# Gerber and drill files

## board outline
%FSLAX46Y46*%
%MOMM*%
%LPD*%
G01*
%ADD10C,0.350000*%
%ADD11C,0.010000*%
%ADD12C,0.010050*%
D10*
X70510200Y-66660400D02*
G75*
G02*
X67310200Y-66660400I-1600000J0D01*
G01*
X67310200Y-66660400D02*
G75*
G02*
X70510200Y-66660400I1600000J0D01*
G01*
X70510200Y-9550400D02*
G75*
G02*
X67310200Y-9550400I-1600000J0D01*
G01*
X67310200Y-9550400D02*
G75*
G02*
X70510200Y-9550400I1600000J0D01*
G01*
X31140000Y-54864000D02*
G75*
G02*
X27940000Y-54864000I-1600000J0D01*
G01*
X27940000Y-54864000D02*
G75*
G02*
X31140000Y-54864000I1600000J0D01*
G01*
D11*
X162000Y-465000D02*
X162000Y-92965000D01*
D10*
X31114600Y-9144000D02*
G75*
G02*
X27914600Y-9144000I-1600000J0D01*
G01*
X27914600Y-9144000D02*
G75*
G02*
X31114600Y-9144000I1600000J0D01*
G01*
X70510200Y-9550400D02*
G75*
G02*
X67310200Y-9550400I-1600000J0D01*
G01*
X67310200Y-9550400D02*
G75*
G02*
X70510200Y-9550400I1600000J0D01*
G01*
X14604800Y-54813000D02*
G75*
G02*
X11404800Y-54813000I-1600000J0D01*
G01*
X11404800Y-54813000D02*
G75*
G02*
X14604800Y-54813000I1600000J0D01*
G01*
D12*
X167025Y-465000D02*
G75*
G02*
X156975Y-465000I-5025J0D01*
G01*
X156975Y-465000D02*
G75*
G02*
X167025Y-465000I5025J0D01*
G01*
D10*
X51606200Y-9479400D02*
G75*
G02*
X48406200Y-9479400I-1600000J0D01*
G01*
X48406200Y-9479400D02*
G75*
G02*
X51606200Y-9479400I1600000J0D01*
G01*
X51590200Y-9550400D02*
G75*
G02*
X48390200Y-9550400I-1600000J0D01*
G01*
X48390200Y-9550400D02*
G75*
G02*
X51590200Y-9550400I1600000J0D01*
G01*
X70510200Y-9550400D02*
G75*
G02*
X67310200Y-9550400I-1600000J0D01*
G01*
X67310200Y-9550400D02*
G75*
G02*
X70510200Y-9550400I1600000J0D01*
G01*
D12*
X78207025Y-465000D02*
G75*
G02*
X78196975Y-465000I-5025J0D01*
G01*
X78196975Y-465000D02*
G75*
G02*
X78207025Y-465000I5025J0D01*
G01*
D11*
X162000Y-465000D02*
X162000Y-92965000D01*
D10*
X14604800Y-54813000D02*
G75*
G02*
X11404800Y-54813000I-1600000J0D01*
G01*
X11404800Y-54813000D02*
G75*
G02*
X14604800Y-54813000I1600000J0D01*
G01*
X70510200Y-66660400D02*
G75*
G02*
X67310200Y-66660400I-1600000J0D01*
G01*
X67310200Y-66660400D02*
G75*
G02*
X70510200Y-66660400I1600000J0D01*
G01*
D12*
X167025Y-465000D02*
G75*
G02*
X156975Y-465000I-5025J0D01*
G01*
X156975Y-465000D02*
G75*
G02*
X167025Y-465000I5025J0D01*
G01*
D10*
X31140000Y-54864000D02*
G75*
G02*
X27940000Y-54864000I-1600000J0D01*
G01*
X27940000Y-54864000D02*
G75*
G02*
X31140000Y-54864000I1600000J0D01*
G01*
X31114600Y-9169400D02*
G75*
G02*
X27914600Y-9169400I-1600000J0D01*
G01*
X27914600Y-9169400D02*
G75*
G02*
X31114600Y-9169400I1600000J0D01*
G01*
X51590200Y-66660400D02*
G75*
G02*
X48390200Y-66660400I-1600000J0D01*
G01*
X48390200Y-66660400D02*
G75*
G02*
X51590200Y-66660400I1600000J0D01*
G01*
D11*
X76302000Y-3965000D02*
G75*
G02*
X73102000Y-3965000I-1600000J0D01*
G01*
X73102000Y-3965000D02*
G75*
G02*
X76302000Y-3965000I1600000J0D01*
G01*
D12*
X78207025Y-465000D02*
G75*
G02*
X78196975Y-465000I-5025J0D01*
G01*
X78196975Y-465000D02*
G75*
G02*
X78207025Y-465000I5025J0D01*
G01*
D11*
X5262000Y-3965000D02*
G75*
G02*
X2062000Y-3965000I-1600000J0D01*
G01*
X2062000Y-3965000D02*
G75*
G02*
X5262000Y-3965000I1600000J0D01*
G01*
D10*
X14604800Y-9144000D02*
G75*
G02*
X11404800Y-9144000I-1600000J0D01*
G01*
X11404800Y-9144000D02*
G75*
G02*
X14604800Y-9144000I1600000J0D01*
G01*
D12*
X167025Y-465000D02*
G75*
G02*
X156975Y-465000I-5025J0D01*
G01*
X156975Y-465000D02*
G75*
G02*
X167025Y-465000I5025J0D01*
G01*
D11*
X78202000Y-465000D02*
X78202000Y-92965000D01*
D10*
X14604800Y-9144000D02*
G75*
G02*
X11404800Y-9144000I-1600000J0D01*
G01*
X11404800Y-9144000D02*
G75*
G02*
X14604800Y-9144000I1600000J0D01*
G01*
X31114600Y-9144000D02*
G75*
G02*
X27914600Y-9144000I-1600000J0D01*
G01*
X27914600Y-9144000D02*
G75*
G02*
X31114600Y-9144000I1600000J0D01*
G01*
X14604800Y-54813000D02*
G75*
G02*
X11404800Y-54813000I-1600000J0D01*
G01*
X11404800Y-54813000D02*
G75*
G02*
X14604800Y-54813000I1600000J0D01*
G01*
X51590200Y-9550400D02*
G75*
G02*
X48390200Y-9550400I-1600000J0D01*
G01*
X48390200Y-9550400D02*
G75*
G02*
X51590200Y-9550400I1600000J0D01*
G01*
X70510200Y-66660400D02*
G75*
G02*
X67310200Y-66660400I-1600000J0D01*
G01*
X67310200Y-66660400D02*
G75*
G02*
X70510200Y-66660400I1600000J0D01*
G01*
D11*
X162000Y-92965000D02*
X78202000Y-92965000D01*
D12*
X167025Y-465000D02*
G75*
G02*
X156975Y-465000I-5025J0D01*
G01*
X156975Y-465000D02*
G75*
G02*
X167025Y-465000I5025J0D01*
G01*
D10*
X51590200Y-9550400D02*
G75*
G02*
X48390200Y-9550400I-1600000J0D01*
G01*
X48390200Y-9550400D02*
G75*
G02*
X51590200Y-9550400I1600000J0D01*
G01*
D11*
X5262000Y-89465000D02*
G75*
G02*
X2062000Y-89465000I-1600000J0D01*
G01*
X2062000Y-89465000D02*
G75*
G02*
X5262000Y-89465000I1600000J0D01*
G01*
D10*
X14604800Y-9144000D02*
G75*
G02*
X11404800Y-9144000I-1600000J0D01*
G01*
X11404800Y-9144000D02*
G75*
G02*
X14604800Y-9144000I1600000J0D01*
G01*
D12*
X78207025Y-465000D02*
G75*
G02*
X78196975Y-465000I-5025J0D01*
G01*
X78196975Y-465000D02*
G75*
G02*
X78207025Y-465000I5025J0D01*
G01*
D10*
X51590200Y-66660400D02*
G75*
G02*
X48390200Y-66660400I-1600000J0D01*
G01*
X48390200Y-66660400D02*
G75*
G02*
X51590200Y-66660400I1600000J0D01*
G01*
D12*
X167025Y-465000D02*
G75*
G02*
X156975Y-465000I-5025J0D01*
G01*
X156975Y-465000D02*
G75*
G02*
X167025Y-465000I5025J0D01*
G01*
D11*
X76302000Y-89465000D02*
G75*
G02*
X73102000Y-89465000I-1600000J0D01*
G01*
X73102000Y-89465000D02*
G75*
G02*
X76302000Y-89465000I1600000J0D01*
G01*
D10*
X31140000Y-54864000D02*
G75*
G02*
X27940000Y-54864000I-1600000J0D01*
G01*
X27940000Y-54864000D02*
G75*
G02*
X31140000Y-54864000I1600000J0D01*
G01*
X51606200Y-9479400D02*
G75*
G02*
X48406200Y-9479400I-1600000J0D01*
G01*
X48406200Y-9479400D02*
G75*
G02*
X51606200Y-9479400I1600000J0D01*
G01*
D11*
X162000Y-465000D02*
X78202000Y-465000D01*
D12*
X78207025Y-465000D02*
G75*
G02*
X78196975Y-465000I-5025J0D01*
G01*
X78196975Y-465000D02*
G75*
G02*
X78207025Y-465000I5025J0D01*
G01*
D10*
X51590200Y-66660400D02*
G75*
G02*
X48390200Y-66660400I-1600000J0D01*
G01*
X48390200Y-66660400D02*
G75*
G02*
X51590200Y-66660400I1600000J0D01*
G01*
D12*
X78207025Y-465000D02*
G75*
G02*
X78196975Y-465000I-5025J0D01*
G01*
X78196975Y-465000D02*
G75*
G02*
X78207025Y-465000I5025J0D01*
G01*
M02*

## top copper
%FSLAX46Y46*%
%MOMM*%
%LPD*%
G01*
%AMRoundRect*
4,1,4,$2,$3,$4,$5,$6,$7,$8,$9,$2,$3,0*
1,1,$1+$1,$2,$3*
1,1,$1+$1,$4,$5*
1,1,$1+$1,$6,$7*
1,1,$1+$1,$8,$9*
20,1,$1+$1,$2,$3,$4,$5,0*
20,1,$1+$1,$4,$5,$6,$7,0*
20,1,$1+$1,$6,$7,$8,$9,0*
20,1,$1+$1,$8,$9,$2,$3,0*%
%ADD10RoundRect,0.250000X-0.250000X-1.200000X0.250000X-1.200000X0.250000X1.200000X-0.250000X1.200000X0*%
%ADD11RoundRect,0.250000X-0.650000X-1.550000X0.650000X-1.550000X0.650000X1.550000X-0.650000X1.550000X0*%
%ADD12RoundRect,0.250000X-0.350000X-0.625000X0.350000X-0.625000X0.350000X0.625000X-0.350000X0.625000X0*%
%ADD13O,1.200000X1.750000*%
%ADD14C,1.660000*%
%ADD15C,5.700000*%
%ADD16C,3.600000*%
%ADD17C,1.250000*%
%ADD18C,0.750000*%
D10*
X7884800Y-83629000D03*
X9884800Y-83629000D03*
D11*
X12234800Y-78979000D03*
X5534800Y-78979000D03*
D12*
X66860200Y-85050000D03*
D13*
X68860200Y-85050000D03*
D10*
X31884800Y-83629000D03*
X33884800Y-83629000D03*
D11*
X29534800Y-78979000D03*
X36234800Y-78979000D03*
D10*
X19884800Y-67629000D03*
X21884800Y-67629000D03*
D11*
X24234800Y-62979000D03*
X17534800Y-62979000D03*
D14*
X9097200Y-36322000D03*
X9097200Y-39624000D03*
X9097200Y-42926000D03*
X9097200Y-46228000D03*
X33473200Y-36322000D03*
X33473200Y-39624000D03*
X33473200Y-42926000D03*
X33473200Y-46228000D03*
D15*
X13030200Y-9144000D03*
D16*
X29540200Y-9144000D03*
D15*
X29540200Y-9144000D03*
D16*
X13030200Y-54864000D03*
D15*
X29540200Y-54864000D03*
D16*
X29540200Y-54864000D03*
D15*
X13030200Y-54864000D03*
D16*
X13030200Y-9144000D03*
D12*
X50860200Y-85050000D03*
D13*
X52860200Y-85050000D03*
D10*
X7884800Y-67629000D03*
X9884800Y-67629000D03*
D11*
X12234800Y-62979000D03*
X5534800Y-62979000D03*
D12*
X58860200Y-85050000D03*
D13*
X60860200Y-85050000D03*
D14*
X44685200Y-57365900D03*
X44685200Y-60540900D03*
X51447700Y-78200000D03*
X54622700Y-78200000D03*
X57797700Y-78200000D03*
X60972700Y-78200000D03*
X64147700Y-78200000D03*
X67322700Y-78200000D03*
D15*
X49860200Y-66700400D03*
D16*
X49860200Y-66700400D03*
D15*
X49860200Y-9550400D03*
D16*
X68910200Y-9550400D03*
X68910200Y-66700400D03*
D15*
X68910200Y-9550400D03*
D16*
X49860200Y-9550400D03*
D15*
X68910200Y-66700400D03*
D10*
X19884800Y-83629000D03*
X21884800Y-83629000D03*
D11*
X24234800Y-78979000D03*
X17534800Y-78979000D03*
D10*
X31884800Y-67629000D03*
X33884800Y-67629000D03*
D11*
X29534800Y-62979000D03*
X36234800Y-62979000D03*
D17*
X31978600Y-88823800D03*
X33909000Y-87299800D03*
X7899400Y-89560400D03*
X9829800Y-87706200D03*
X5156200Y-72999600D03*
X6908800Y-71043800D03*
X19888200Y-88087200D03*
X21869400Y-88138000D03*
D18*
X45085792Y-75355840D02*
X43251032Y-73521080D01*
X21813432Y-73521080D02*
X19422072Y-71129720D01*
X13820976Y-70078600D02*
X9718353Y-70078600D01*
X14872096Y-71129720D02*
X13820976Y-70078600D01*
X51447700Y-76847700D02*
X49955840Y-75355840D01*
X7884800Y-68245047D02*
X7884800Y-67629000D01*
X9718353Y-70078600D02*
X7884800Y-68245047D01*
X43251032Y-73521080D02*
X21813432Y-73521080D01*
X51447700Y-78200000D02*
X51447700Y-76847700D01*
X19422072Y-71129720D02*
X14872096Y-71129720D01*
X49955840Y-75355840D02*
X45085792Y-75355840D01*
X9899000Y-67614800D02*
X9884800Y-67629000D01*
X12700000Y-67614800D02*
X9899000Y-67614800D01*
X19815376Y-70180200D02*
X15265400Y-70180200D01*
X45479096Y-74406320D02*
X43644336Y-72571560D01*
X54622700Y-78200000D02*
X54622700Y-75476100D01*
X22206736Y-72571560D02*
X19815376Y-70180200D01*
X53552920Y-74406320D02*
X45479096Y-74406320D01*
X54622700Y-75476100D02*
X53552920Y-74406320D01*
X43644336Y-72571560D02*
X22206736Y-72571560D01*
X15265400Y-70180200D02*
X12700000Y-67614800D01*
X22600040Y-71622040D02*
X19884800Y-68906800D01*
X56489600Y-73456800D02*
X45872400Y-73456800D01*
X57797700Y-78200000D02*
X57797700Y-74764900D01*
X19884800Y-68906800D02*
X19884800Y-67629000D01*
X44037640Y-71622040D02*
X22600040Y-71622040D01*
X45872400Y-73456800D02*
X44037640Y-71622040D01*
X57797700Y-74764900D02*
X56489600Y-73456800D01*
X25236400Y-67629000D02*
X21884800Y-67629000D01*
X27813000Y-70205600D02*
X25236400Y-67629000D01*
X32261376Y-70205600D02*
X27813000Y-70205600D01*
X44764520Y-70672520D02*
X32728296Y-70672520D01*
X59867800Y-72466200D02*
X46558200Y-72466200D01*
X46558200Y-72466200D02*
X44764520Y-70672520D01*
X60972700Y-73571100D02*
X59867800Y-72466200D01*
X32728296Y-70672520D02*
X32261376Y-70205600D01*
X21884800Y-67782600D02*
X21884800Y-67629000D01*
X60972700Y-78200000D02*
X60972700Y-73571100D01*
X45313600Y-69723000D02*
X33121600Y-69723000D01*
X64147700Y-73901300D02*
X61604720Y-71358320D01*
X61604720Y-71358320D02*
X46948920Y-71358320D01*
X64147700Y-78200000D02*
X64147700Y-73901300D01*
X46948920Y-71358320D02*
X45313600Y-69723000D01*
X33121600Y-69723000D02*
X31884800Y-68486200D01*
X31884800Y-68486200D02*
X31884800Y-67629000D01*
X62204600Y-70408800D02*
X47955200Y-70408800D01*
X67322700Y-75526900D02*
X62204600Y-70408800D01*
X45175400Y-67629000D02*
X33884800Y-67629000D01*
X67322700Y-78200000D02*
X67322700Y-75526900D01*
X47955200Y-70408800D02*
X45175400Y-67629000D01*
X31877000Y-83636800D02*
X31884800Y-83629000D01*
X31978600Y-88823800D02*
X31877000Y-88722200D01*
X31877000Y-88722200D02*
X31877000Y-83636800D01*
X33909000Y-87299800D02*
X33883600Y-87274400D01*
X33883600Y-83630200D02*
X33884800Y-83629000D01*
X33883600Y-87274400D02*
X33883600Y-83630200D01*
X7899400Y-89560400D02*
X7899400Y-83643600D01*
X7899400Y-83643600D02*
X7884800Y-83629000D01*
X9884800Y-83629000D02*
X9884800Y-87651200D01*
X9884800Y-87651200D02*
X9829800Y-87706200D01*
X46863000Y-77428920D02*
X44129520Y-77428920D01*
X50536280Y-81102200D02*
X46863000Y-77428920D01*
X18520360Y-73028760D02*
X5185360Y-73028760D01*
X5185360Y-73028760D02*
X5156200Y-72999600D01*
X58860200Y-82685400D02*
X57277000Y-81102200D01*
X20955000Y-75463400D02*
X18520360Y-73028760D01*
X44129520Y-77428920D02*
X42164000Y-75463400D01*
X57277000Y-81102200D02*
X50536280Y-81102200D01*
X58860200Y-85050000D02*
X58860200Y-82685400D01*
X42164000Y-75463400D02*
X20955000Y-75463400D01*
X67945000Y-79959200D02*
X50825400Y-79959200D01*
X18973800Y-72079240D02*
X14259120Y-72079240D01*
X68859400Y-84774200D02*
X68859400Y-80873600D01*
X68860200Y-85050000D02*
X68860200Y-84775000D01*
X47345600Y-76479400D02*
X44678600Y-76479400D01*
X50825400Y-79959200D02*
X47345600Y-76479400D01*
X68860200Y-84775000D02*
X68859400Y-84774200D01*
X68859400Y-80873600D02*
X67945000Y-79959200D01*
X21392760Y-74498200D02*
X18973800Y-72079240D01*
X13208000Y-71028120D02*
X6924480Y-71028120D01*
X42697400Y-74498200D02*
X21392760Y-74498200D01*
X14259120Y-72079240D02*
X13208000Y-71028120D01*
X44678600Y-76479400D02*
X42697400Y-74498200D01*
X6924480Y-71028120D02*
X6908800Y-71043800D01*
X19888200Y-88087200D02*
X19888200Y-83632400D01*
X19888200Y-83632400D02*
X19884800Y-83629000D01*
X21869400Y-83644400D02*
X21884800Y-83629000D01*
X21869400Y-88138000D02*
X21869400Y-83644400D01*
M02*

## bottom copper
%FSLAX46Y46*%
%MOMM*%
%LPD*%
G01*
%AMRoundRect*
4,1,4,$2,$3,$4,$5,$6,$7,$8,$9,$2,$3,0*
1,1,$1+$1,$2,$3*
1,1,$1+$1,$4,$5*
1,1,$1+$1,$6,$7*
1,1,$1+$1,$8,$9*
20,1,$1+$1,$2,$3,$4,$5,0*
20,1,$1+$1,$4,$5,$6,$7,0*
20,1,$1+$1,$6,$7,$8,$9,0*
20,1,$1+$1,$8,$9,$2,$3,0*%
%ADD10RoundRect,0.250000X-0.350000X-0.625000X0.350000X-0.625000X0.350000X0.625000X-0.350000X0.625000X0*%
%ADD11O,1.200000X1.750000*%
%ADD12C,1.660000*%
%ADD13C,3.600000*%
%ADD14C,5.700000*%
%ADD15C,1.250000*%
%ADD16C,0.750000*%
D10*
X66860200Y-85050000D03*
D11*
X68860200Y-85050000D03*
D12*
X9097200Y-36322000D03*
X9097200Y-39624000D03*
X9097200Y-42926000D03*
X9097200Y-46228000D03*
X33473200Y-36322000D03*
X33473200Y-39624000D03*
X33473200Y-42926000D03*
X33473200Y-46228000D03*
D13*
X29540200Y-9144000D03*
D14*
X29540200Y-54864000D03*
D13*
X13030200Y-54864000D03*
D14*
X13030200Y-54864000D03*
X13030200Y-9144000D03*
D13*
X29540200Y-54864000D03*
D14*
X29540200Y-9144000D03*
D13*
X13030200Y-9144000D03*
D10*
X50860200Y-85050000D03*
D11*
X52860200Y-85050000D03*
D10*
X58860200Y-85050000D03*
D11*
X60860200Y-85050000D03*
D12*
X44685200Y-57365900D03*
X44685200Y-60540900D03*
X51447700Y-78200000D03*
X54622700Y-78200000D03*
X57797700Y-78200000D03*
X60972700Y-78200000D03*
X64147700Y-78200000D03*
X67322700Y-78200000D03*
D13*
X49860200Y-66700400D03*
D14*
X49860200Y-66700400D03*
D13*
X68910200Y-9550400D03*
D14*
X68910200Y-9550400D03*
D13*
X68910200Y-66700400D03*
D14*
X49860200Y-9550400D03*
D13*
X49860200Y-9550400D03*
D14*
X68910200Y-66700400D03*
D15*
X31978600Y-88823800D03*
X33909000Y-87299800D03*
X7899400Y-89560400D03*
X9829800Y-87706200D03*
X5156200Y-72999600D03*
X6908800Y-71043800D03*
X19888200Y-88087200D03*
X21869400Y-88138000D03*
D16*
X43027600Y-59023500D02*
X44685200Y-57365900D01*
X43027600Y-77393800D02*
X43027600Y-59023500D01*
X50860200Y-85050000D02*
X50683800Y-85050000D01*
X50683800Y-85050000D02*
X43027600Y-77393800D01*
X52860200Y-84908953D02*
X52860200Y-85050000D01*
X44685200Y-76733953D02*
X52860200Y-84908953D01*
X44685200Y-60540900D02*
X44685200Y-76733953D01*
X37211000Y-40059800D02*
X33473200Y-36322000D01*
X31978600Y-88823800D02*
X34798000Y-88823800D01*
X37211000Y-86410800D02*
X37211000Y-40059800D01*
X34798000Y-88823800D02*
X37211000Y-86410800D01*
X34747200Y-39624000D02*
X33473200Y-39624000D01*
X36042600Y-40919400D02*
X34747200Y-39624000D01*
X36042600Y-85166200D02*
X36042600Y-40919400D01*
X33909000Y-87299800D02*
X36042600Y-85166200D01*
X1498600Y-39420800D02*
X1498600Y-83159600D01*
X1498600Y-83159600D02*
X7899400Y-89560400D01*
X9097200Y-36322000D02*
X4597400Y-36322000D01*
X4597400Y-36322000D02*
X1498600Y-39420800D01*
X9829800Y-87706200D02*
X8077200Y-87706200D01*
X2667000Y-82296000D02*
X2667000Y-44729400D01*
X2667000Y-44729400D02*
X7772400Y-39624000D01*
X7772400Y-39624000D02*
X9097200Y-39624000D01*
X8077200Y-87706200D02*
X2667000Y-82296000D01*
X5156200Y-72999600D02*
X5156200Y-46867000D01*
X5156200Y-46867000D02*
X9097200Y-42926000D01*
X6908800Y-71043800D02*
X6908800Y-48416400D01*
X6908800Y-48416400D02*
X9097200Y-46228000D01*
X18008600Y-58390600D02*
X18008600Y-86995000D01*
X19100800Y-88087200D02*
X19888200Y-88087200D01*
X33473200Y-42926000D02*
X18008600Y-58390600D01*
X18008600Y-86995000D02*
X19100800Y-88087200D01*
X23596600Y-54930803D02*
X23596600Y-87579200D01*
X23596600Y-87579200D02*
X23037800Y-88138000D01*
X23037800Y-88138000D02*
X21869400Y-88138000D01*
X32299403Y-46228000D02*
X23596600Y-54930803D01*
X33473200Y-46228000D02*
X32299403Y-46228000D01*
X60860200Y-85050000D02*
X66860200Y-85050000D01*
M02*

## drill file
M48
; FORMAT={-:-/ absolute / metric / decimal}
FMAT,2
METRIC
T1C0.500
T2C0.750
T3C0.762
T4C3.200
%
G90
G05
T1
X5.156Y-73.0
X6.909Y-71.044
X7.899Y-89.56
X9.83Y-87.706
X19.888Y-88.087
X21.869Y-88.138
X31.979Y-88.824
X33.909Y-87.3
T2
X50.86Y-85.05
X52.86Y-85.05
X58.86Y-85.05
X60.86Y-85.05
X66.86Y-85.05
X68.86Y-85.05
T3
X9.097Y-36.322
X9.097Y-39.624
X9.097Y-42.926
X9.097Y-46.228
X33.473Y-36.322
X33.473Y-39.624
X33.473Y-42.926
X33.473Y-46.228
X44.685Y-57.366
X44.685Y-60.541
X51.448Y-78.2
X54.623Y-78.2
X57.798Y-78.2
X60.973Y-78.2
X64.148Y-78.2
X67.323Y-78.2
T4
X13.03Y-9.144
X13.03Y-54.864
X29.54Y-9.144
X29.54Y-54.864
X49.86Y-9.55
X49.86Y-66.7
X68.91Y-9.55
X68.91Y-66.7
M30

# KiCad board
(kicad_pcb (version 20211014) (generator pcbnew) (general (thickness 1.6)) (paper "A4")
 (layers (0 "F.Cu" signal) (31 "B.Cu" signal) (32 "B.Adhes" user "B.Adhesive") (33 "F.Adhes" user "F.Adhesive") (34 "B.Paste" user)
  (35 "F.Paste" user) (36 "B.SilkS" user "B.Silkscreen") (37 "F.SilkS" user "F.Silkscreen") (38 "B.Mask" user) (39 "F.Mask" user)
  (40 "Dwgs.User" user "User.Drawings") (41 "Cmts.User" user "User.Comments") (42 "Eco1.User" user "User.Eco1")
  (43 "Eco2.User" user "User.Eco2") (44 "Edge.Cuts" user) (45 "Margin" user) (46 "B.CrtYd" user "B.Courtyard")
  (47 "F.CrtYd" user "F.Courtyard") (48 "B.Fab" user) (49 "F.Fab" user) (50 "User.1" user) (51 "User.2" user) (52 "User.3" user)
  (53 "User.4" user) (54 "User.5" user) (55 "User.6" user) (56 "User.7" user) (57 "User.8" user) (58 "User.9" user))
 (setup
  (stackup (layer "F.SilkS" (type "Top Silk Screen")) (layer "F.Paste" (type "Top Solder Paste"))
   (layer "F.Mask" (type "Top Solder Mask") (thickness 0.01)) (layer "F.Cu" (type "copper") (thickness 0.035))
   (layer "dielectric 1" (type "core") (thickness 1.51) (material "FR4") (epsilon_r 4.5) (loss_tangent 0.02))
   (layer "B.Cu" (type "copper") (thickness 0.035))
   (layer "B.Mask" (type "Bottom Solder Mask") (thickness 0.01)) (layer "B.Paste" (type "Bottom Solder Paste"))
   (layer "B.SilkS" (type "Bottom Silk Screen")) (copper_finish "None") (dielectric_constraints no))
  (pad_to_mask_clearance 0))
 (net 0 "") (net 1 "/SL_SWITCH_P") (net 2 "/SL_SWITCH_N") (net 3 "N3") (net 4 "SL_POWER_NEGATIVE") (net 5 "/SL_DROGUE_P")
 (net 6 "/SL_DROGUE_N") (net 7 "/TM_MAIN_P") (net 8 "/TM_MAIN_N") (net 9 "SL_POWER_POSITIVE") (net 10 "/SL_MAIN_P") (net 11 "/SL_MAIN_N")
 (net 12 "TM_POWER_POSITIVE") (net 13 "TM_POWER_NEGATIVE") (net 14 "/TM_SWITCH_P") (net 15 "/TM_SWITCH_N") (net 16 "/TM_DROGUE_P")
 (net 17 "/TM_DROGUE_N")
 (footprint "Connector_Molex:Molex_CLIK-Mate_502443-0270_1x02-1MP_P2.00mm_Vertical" (layer "F.Cu") (at 8.8848 81.129)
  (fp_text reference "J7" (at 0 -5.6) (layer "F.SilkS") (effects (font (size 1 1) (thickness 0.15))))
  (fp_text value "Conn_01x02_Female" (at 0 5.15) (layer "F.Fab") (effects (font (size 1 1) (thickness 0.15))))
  (pad "1" smd roundrect (at -1 2.5) (size 1 2.9) (layers "F.Cu" "F.Paste" "F.Mask") (roundrect_rratio 0.25) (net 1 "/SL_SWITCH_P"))
  (pad "2" smd roundrect (at 1 2.5) (size 1 2.9) (layers "F.Cu" "F.Paste" "F.Mask") (roundrect_rratio 0.25) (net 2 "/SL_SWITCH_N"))
  (pad "MP" smd roundrect (at 3.35 -2.15) (size 1.8 3.6) (layers "F.Cu" "F.Paste" "F.Mask") (roundrect_rratio 0.138889))
  (pad "MP" smd roundrect (at -3.35 -2.15) (size 1.8 3.6) (layers "F.Cu" "F.Paste" "F.Mask") (roundrect_rratio 0.138889)))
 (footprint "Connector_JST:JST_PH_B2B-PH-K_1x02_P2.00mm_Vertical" (layer "F.Cu") (at 66.8602 85.05)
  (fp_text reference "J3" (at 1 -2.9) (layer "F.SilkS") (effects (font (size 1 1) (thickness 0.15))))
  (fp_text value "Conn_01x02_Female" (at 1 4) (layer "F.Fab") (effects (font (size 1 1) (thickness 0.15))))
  (pad "1" thru_hole roundrect (at 0 0) (size 1.2 1.75) (drill 0.75) (layers *.Cu *.Mask) (roundrect_rratio 0.208333) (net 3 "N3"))
  (pad "2" thru_hole oval (at 2 0) (size 1.2 1.75) (drill 0.75) (layers *.Cu *.Mask) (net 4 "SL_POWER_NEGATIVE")))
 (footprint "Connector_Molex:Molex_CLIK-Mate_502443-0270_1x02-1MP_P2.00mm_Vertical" (layer "F.Cu") (at 32.8848 81.129)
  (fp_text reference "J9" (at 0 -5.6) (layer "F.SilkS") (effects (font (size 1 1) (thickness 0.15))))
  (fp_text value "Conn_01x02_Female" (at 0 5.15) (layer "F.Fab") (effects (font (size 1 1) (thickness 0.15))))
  (pad "1" smd roundrect (at -1 2.5) (size 1 2.9) (layers "F.Cu" "F.Paste" "F.Mask") (roundrect_rratio 0.25) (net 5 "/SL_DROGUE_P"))
  (pad "2" smd roundrect (at 1 2.5) (size 1 2.9) (layers "F.Cu" "F.Paste" "F.Mask") (roundrect_rratio 0.25) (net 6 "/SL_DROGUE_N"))
  (pad "MP" smd roundrect (at -3.35 -2.15) (size 1.8 3.6) (layers "F.Cu" "F.Paste" "F.Mask") (roundrect_rratio 0.138889))
  (pad "MP" smd roundrect (at 3.35 -2.15) (size 1.8 3.6) (layers "F.Cu" "F.Paste" "F.Mask") (roundrect_rratio 0.138889)))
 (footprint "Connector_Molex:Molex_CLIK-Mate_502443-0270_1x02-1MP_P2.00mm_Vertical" (layer "F.Cu") (at 20.8848 65.129)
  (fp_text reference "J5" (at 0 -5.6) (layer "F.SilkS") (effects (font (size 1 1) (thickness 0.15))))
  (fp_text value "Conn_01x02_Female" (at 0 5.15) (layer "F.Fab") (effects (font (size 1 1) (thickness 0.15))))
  (pad "1" smd roundrect (at -1 2.5) (size 1 2.9) (layers "F.Cu" "F.Paste" "F.Mask") (roundrect_rratio 0.25) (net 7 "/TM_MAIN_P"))
  (pad "2" smd roundrect (at 1 2.5) (size 1 2.9) (layers "F.Cu" "F.Paste" "F.Mask") (roundrect_rratio 0.25) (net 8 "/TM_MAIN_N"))
  (pad "MP" smd roundrect (at 3.35 -2.15) (size 1.8 3.6) (layers "F.Cu" "F.Paste" "F.Mask") (roundrect_rratio 0.138889))
  (pad "MP" smd roundrect (at -3.35 -2.15) (size 1.8 3.6) (layers "F.Cu" "F.Paste" "F.Mask") (roundrect_rratio 0.138889)))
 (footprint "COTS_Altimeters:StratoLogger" (layer "F.Cu") (at 21.2852 32.004 -90)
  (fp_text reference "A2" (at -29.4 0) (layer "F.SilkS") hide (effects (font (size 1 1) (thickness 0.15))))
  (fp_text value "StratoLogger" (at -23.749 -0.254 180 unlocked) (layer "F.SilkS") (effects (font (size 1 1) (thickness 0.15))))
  (pad "1" thru_hole circle locked (at 4.318 12.188 270) (size 1.66 1.66) (drill 0.762) (layers *.Cu *.Mask) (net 1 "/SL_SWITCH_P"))
  (pad "2" thru_hole circle locked (at 7.62 12.188 270) (size 1.66 1.66) (drill 0.762) (layers *.Cu *.Mask) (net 2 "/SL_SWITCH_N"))
  (pad "3" thru_hole circle locked (at 10.922 12.188 270) (size 1.66 1.66) (drill 0.762) (layers *.Cu *.Mask) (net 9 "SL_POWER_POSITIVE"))
  (pad "4" thru_hole circle locked (at 14.224 12.188 270) (size 1.66 1.66) (drill 0.762) (layers *.Cu *.Mask) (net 4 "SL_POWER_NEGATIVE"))
  (pad "5" thru_hole circle locked (at 4.318 -12.188 270) (size 1.66 1.66) (drill 0.762) (layers *.Cu *.Mask) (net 5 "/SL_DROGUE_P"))
  (pad "6" thru_hole circle locked (at 7.62 -12.188 270) (size 1.66 1.66) (drill 0.762) (layers *.Cu *.Mask) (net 6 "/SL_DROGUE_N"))
  (pad "7" thru_hole circle locked (at 10.922 -12.188 270) (size 1.66 1.66) (drill 0.762) (layers *.Cu *.Mask) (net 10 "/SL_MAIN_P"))
  (pad "8" thru_hole circle locked (at 14.224 -12.188 270) (size 1.66 1.66) (drill 0.762) (layers *.Cu *.Mask) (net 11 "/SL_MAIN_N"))
  (pad "~" connect circle locked (at -22.86 8.255 270) (size 5.7 5.7) (layers "F.Cu" "F.Mask"))
  (pad "~" thru_hole circle locked (at -22.86 -8.255 270) (size 3.6 3.6) (drill 3.2) (layers *.Cu *.Mask))
  (pad "~" connect circle locked (at 22.86 -8.255 270) (size 5.7 5.7) (layers "B.Cu" "B.Mask"))
  (pad "~" connect circle locked (at -22.86 -8.255 270) (size 5.7 5.7) (layers "F.Cu" "F.Mask"))
  (pad "~" thru_hole circle locked (at 22.86 8.255 270) (size 3.6 3.6) (drill 3.2) (layers *.Cu *.Mask))
  (pad "~" connect circle locked (at 22.86 8.255 270) (size 5.7 5.7) (layers "B.Cu" "B.Mask"))
  (pad "~" connect circle locked (at -22.86 8.255 270) (size 5.7 5.7) (layers "B.Cu" "B.Mask"))
  (pad "~" connect circle locked (at 22.86 -8.255 270) (size 5.7 5.7) (layers "F.Cu" "F.Mask"))
  (pad "~" thru_hole circle locked (at 22.86 -8.255 270) (size 3.6 3.6) (drill 3.2) (layers *.Cu *.Mask))
  (pad "~" connect circle locked (at -22.86 -8.255 270) (size 5.7 5.7) (layers "B.Cu" "B.Mask"))
  (pad "~" connect circle locked (at 22.86 8.255 270) (size 5.7 5.7) (layers "F.Cu" "F.Mask"))
  (pad "~" thru_hole circle locked (at -22.86 8.255 270) (size 3.6 3.6) (drill 3.2) (layers *.Cu *.Mask)))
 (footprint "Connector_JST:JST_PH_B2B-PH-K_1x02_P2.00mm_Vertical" (layer "F.Cu") (at 50.8602 85.05)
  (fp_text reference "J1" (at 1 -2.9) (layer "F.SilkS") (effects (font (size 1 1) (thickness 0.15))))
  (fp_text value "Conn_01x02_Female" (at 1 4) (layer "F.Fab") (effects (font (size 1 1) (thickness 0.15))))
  (pad "1" thru_hole roundrect (at 0 0) (size 1.2 1.75) (drill 0.75) (layers *.Cu *.Mask) (roundrect_rratio 0.208333)
   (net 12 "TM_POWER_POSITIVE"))
  (pad "2" thru_hole oval (at 2 0) (size 1.2 1.75) (drill 0.75) (layers *.Cu *.Mask) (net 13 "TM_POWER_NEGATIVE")))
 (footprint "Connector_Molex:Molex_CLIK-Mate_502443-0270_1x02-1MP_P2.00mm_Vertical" (layer "F.Cu") (at 8.8848 65.129)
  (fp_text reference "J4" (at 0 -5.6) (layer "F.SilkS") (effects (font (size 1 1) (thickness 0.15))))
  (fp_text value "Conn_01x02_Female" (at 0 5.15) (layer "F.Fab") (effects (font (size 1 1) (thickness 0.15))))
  (pad "1" smd roundrect (at -1 2.5) (size 1 2.9) (layers "F.Cu" "F.Paste" "F.Mask") (roundrect_rratio 0.25) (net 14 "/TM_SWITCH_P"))
  (pad "2" smd roundrect (at 1 2.5) (size 1 2.9) (layers "F.Cu" "F.Paste" "F.Mask") (roundrect_rratio 0.25) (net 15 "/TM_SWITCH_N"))
  (pad "MP" smd roundrect (at 3.35 -2.15) (size 1.8 3.6) (layers "F.Cu" "F.Paste" "F.Mask") (roundrect_rratio 0.138889))
  (pad "MP" smd roundrect (at -3.35 -2.15) (size 1.8 3.6) (layers "F.Cu" "F.Paste" "F.Mask") (roundrect_rratio 0.138889)))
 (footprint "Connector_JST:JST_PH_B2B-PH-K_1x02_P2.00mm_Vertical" (layer "F.Cu") (at 58.8602 85.05)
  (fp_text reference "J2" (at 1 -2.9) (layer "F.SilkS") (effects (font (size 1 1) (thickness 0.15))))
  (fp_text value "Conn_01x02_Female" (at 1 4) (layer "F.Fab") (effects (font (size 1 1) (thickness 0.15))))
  (pad "1" thru_hole roundrect (at 0 0) (size 1.2 1.75) (drill 0.75) (layers *.Cu *.Mask) (roundrect_rratio 0.208333)
   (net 9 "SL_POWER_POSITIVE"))
  (pad "2" thru_hole oval (at 2 0) (size 1.2 1.75) (drill 0.75) (layers *.Cu *.Mask) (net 3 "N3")))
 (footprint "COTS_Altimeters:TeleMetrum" (layer "F.Cu") (at 59.3852 41.275 90)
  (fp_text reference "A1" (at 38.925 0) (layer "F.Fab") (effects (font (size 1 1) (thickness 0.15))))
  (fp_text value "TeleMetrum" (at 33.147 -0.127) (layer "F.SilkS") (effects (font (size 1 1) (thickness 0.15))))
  (pad "1" thru_hole circle locked (at -16.0909 -14.7 90) (size 1.66 1.66) (drill 0.762) (layers *.Cu *.Mask) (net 12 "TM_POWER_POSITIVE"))
  (pad "2" thru_hole circle locked (at -19.2659 -14.7 90) (size 1.66 1.66) (drill 0.762) (layers *.Cu *.Mask) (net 13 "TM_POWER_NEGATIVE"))
  (pad "3" thru_hole circle locked (at -36.925 -7.9375 90) (size 1.66 1.66) (drill 0.762) (layers *.Cu *.Mask) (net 14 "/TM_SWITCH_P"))
  (pad "4" thru_hole circle locked (at -36.925 -4.7625 90) (size 1.66 1.66) (drill 0.762) (layers *.Cu *.Mask) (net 15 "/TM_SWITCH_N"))
  (pad "5" thru_hole circle locked (at -36.925 -1.5875 90) (size 1.66 1.66) (drill 0.762) (layers *.Cu *.Mask) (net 7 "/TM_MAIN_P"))
  (pad "6" thru_hole circle locked (at -36.925 1.5875 90) (size 1.66 1.66) (drill 0.762) (layers *.Cu *.Mask) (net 8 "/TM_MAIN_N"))
  (pad "7" thru_hole circle locked (at -36.925 4.7625 90) (size 1.66 1.66) (drill 0.762) (layers *.Cu *.Mask) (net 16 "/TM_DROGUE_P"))
  (pad "8" thru_hole circle locked (at -36.925 7.9375 90) (size 1.66 1.66) (drill 0.762) (layers *.Cu *.Mask) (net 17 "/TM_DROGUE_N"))
  (pad "~" connect circle locked (at -25.4254 -9.525 90) (size 5.7 5.7) (layers "F.Cu" "F.Mask"))
  (pad "~" thru_hole circle locked (at -25.4254 -9.525 90) (size 3.6 3.6) (drill 3.2) (layers *.Cu *.Mask))
  (pad "~" connect circle locked (at -25.4254 -9.525 90) (size 5.7 5.7) (layers "B.Cu" "B.Mask"))
  (pad "~" connect circle locked (at 31.7246 -9.525 90) (size 5.7 5.7) (layers "F.Cu" "F.Mask"))
  (pad "~" thru_hole circle locked (at 31.7246 9.525 90) (size 3.6 3.6) (drill 3.2) (layers *.Cu *.Mask))
  (pad "~" connect circle locked (at 31.7246 9.525 90) (size 5.7 5.7) (layers "B.Cu" "B.Mask"))
  (pad "~" thru_hole circle locked (at -25.4254 9.525 90) (size 3.6 3.6) (drill 3.2) (layers *.Cu *.Mask))
  (pad "~" connect circle locked (at 31.7246 9.525 90) (size 5.7 5.7) (layers "F.Cu" "F.Mask"))
  (pad "~" connect circle locked (at 31.7246 -9.525 90) (size 5.7 5.7) (layers "B.Cu" "B.Mask"))
  (pad "~" thru_hole circle locked (at 31.7246 -9.525 90) (size 3.6 3.6) (drill 3.2) (layers *.Cu *.Mask))
  (pad "~" connect circle locked (at -25.4254 9.525 90) (size 5.7 5.7) (layers "F.Cu" "F.Mask"))
  (pad "~" connect circle locked (at -25.4254 9.525 90) (size 5.7 5.7) (layers "B.Cu" "B.Mask")))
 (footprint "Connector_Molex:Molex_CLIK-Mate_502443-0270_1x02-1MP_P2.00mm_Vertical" (layer "F.Cu") (at 20.8848 81.129)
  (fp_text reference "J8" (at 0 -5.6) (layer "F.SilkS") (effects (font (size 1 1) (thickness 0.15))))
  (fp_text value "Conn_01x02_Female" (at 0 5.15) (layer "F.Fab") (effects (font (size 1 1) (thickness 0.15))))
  (pad "1" smd roundrect (at -1 2.5) (size 1 2.9) (layers "F.Cu" "F.Paste" "F.Mask") (roundrect_rratio 0.25) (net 10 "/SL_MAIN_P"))
  (pad "2" smd roundrect (at 1 2.5) (size 1 2.9) (layers "F.Cu" "F.Paste" "F.Mask") (roundrect_rratio 0.25) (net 11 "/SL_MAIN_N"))
  (pad "MP" smd roundrect (at 3.35 -2.15) (size 1.8 3.6) (layers "F.Cu" "F.Paste" "F.Mask") (roundrect_rratio 0.138889))
  (pad "MP" smd roundrect (at -3.35 -2.15) (size 1.8 3.6) (layers "F.Cu" "F.Paste" "F.Mask") (roundrect_rratio 0.138889)))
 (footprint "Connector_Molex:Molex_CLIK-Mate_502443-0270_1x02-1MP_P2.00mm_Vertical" (layer "F.Cu") (at 32.8848 65.129)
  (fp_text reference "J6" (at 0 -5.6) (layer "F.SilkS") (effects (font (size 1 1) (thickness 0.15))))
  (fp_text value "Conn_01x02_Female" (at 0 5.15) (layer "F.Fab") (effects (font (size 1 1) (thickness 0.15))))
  (pad "1" smd roundrect (at -1 2.5) (size 1 2.9) (layers "F.Cu" "F.Paste" "F.Mask") (roundrect_rratio 0.25) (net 16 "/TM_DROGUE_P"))
  (pad "2" smd roundrect (at 1 2.5) (size 1 2.9) (layers "F.Cu" "F.Paste" "F.Mask") (roundrect_rratio 0.25) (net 17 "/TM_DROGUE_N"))
  (pad "MP" smd roundrect (at -3.35 -2.15) (size 1.8 3.6) (layers "F.Cu" "F.Paste" "F.Mask") (roundrect_rratio 0.138889))
  (pad "MP" smd roundrect (at 3.35 -2.15) (size 1.8 3.6) (layers "F.Cu" "F.Paste" "F.Mask") (roundrect_rratio 0.138889)))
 (gr_circle (center 68.9102 66.6604) (end 70.5102 66.6604) (layer "Edge.Cuts") (width 0.35) (fill none))
 (gr_circle (center 68.9102 9.5504) (end 70.5102 9.5504) (layer "Edge.Cuts") (width 0.35) (fill none))
 (gr_circle (center 29.54 54.864) (end 31.14 54.864) (layer "Edge.Cuts") (width 0.35) (fill none))
 (gr_line (start 0.162 0.465) (end 0.162 92.965) (layer "Edge.Cuts") (width 0.01))
 (gr_circle (center 29.5146 9.144) (end 31.1146 9.144) (layer "Edge.Cuts") (width 0.35) (fill none))
 (gr_circle (center 68.9102 9.5504) (end 70.5102 9.5504) (layer "Edge.Cuts") (width 0.35) (fill none))
 (gr_circle (center 13.0048 54.813) (end 14.6048 54.813) (layer "Edge.Cuts") (width 0.35) (fill none))
 (gr_circle (center 0.162 0.465) (end 0.172 0.465) (layer "Edge.Cuts") (width 0.0001) (fill solid))
 (gr_circle (center 50.0062 9.4794) (end 51.6062 9.4794) (layer "Edge.Cuts") (width 0.35) (fill none))
 (gr_circle (center 49.9902 9.5504) (end 51.5902 9.5504) (layer "Edge.Cuts") (width 0.35) (fill none))
 (gr_circle (center 68.9102 9.5504) (end 70.5102 9.5504) (layer "Edge.Cuts") (width 0.35) (fill none))
 (gr_circle (center 78.202 0.465) (end 78.212 0.465) (layer "Edge.Cuts") (width 0.0001) (fill solid))
 (gr_line (start 0.162 0.465) (end 0.162 92.965) (layer "Edge.Cuts") (width 0.01))
 (gr_circle (center 13.0048 54.813) (end 14.6048 54.813) (layer "Edge.Cuts") (width 0.35) (fill none))
 (gr_circle (center 68.9102 66.6604) (end 70.5102 66.6604) (layer "Edge.Cuts") (width 0.35) (fill none))
 (gr_circle (center 0.162 0.465) (end 0.172 0.465) (layer "Edge.Cuts") (width 0.0001) (fill solid))
 (gr_circle (center 29.54 54.864) (end 31.14 54.864) (layer "Edge.Cuts") (width 0.35) (fill none))
 (gr_circle (center 29.5146 9.1694) (end 31.1146 9.1694) (layer "Edge.Cuts") (width 0.35) (fill none))
 (gr_circle (center 49.9902 66.6604) (end 51.5902 66.6604) (layer "Edge.Cuts") (width 0.35) (fill none))
 (gr_circle (center 74.702 3.965) (end 76.302 3.965) (layer "Edge.Cuts") (width 0.01) (fill none))
 (gr_circle (center 78.202 0.465) (end 78.212 0.465) (layer "Edge.Cuts") (width 0.0001) (fill solid))
 (gr_circle (center 3.662 3.965) (end 5.262 3.965) (layer "Edge.Cuts") (width 0.01) (fill none))
 (gr_circle (center 13.0048 9.144) (end 14.6048 9.144) (layer "Edge.Cuts") (width 0.35) (fill none))
 (gr_circle (center 0.162 0.465) (end 0.172 0.465) (layer "Edge.Cuts") (width 0.0001) (fill solid))
 (gr_line (start 78.202 0.465) (end 78.202 92.965) (layer "Edge.Cuts") (width 0.01))
 (gr_circle (center 13.0048 9.144) (end 14.6048 9.144) (layer "Edge.Cuts") (width 0.35) (fill none))
 (gr_circle (center 29.5146 9.144) (end 31.1146 9.144) (layer "Edge.Cuts") (width 0.35) (fill none))
 (gr_circle (center 13.0048 54.813) (end 14.6048 54.813) (layer "Edge.Cuts") (width 0.35) (fill none))
 (gr_circle (center 49.9902 9.5504) (end 51.5902 9.5504) (layer "Edge.Cuts") (width 0.35) (fill none))
 (gr_circle (center 68.9102 66.6604) (end 70.5102 66.6604) (layer "Edge.Cuts") (width 0.35) (fill none))
 (gr_line (start 0.162 92.965) (end 78.202 92.965) (layer "Edge.Cuts") (width 0.01))
 (gr_circle (center 0.162 0.465) (end 0.172 0.465) (layer "Edge.Cuts") (width 0.0001) (fill solid))
 (gr_circle (center 49.9902 9.5504) (end 51.5902 9.5504) (layer "Edge.Cuts") (width 0.35) (fill none))
 (gr_circle (center 3.662 89.465) (end 5.262 89.465) (layer "Edge.Cuts") (width 0.01) (fill none))
 (gr_circle (center 13.0048 9.144) (end 14.6048 9.144) (layer "Edge.Cuts") (width 0.35) (fill none))
 (gr_circle (center 78.202 0.465) (end 78.212 0.465) (layer "Edge.Cuts") (width 0.0001) (fill solid))
 (gr_circle (center 49.9902 66.6604) (end 51.5902 66.6604) (layer "Edge.Cuts") (width 0.35) (fill none))
 (gr_circle (center 0.162 0.465) (end 0.172 0.465) (layer "Edge.Cuts") (width 0.0001) (fill solid))
 (gr_circle (center 74.702 89.465) (end 76.302 89.465) (layer "Edge.Cuts") (width 0.01) (fill none))
 (gr_circle (center 29.54 54.864) (end 31.14 54.864) (layer "Edge.Cuts") (width 0.35) (fill none))
 (gr_circle (center 50.0062 9.4794) (end 51.6062 9.4794) (layer "Edge.Cuts") (width 0.35) (fill none))
 (gr_line (start 0.162 0.465) (end 78.202 0.465) (layer "Edge.Cuts") (width 0.01))
 (gr_circle (center 78.202 0.465) (end 78.212 0.465) (layer "Edge.Cuts") (width 0.0001) (fill solid))
 (gr_circle (center 49.9902 66.6604) (end 51.5902 66.6604) (layer "Edge.Cuts") (width 0.35) (fill none))
 (gr_circle (center 78.202 0.465) (end 78.212 0.465) (layer "Edge.Cuts") (width 0.0001) (fill solid))
 (segment (start 45.085792 75.35584) (end 43.251032 73.52108) (width 0.75) (layer "F.Cu") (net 14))
 (segment (start 21.813432 73.52108) (end 19.422072 71.12972) (width 0.75) (layer "F.Cu") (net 14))
 (segment (start 13.820976 70.0786) (end 9.718353 70.0786) (width 0.75) (layer "F.Cu") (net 14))
 (segment (start 14.872096 71.12972) (end 13.820976 70.0786) (width 0.75) (layer "F.Cu") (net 14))
 (segment (start 51.4477 76.8477) (end 49.95584 75.35584) (width 0.75) (layer "F.Cu") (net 14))
 (segment (start 7.8848 68.245047) (end 7.8848 67.629) (width 0.75) (layer "F.Cu") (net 14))
 (segment (start 9.718353 70.0786) (end 7.8848 68.245047) (width 0.75) (layer "F.Cu") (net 14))
 (segment (start 43.251032 73.52108) (end 21.813432 73.52108) (width 0.75) (layer "F.Cu") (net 14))
 (segment (start 51.4477 78.2) (end 51.4477 76.8477) (width 0.75) (layer "F.Cu") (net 14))
 (segment (start 19.422072 71.12972) (end 14.872096 71.12972) (width 0.75) (layer "F.Cu") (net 14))
 (segment (start 49.95584 75.35584) (end 45.085792 75.35584) (width 0.75) (layer "F.Cu") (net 14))
 (segment (start 9.899 67.6148) (end 9.8848 67.629) (width 0.75) (layer "F.Cu") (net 15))
 (segment (start 12.7 67.6148) (end 9.899 67.6148) (width 0.75) (layer "F.Cu") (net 15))
 (segment (start 19.815376 70.1802) (end 15.2654 70.1802) (width 0.75) (layer "F.Cu") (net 15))
 (segment (start 45.479096 74.40632) (end 43.644336 72.57156) (width 0.75) (layer "F.Cu") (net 15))
 (segment (start 54.6227 78.2) (end 54.6227 75.4761) (width 0.75) (layer "F.Cu") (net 15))
 (segment (start 22.206736 72.57156) (end 19.815376 70.1802) (width 0.75) (layer "F.Cu") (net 15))
 (segment (start 53.55292 74.40632) (end 45.479096 74.40632) (width 0.75) (layer "F.Cu") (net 15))
 (segment (start 54.6227 75.4761) (end 53.55292 74.40632) (width 0.75) (layer "F.Cu") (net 15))
 (segment (start 43.644336 72.57156) (end 22.206736 72.57156) (width 0.75) (layer "F.Cu") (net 15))
 (segment (start 15.2654 70.1802) (end 12.7 67.6148) (width 0.75) (layer "F.Cu") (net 15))
 (segment (start 22.60004 71.62204) (end 19.8848 68.9068) (width 0.75) (layer "F.Cu") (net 7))
 (segment (start 56.4896 73.4568) (end 45.8724 73.4568) (width 0.75) (layer "F.Cu") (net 7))
 (segment (start 57.7977 78.2) (end 57.7977 74.7649) (width 0.75) (layer "F.Cu") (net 7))
 (segment (start 19.8848 68.9068) (end 19.8848 67.629) (width 0.75) (layer "F.Cu") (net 7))
 (segment (start 44.03764 71.62204) (end 22.60004 71.62204) (width 0.75) (layer "F.Cu") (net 7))
 (segment (start 45.8724 73.4568) (end 44.03764 71.62204) (width 0.75) (layer "F.Cu") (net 7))
 (segment (start 57.7977 74.7649) (end 56.4896 73.4568) (width 0.75) (layer "F.Cu") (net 7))
 (segment (start 25.2364 67.629) (end 21.8848 67.629) (width 0.75) (layer "F.Cu") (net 8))
 (segment (start 27.813 70.2056) (end 25.2364 67.629) (width 0.75) (layer "F.Cu") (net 8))
 (segment (start 32.261376 70.2056) (end 27.813 70.2056) (width 0.75) (layer "F.Cu") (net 8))
 (segment (start 44.76452 70.67252) (end 32.728296 70.67252) (width 0.75) (layer "F.Cu") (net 8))
 (segment (start 59.8678 72.4662) (end 46.5582 72.4662) (width 0.75) (layer "F.Cu") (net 8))
 (segment (start 46.5582 72.4662) (end 44.76452 70.67252) (width 0.75) (layer "F.Cu") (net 8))
 (segment (start 60.9727 73.5711) (end 59.8678 72.4662) (width 0.75) (layer "F.Cu") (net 8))
 (segment (start 32.728296 70.67252) (end 32.261376 70.2056) (width 0.75) (layer "F.Cu") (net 8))
 (segment (start 21.8848 67.7826) (end 21.8848 67.629) (width 0.75) (layer "F.Cu") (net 8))
 (segment (start 60.9727 78.2) (end 60.9727 73.5711) (width 0.75) (layer "F.Cu") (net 8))
 (segment (start 45.3136 69.723) (end 33.1216 69.723) (width 0.75) (layer "F.Cu") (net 16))
 (segment (start 64.1477 73.9013) (end 61.60472 71.35832) (width 0.75) (layer "F.Cu") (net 16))
 (segment (start 61.60472 71.35832) (end 46.94892 71.35832) (width 0.75) (layer "F.Cu") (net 16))
 (segment (start 64.1477 78.2) (end 64.1477 73.9013) (width 0.75) (layer "F.Cu") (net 16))
 (segment (start 46.94892 71.35832) (end 45.3136 69.723) (width 0.75) (layer "F.Cu") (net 16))
 (segment (start 33.1216 69.723) (end 31.8848 68.4862) (width 0.75) (layer "F.Cu") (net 16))
 (segment (start 31.8848 68.4862) (end 31.8848 67.629) (width 0.75) (layer "F.Cu") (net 16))
 (segment (start 62.2046 70.4088) (end 47.9552 70.4088) (width 0.75) (layer "F.Cu") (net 17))
 (segment (start 67.3227 75.5269) (end 62.2046 70.4088) (width 0.75) (layer "F.Cu") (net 17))
 (segment (start 45.1754 67.629) (end 33.8848 67.629) (width 0.75) (layer "F.Cu") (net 17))
 (segment (start 67.3227 78.2) (end 67.3227 75.5269) (width 0.75) (layer "F.Cu") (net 17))
 (segment (start 47.9552 70.4088) (end 45.1754 67.629) (width 0.75) (layer "F.Cu") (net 17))
 (segment (start 43.0276 59.0235) (end 44.6852 57.3659) (width 0.75) (layer "B.Cu") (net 12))
 (segment (start 43.0276 77.3938) (end 43.0276 59.0235) (width 0.75) (layer "B.Cu") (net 12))
 (segment (start 50.8602 85.05) (end 50.6838 85.05) (width 0.75) (layer "B.Cu") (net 12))
 (segment (start 50.6838 85.05) (end 43.0276 77.3938) (width 0.75) (layer "B.Cu") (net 12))
 (segment (start 52.8602 84.908953) (end 52.8602 85.05) (width 0.75) (layer "B.Cu") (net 13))
 (segment (start 44.6852 76.733953) (end 52.8602 84.908953) (width 0.75) (layer "B.Cu") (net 13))
 (segment (start 44.6852 60.5409) (end 44.6852 76.733953) (width 0.75) (layer "B.Cu") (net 13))
 (segment (start 31.877 83.6368) (end 31.8848 83.629) (width 0.75) (layer "F.Cu") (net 5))
 (segment (start 31.9786 88.8238) (end 31.877 88.7222) (width 0.75) (layer "F.Cu") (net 5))
 (segment (start 31.877 88.7222) (end 31.877 83.6368) (width 0.75) (layer "F.Cu") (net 5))
 (via (at 31.9786 88.8238) (size 1.25) (drill 0.5) (layers "F.Cu" "B.Cu") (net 5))
 (segment (start 37.211 40.0598) (end 33.4732 36.322) (width 0.75) (layer "B.Cu") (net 5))
 (segment (start 31.9786 88.8238) (end 34.798 88.8238) (width 0.75) (layer "B.Cu") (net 5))
 (segment (start 37.211 86.4108) (end 37.211 40.0598) (width 0.75) (layer "B.Cu") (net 5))
 (segment (start 34.798 88.8238) (end 37.211 86.4108) (width 0.75) (layer "B.Cu") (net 5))
 (segment (start 33.909 87.2998) (end 33.8836 87.2744) (width 0.75) (layer "F.Cu") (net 6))
 (segment (start 33.8836 83.6302) (end 33.8848 83.629) (width 0.75) (layer "F.Cu") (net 6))
 (segment (start 33.8836 87.2744) (end 33.8836 83.6302) (width 0.75) (layer "F.Cu") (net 6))
 (via (at 33.909 87.2998) (size 1.25) (drill 0.5) (layers "F.Cu" "B.Cu") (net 6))
 (segment (start 34.7472 39.624) (end 33.4732 39.624) (width 0.75) (layer "B.Cu") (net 6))
 (segment (start 36.0426 40.9194) (end 34.7472 39.624) (width 0.75) (layer "B.Cu") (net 6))
 (segment (start 36.0426 85.1662) (end 36.0426 40.9194) (width 0.75) (layer "B.Cu") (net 6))
 (segment (start 33.909 87.2998) (end 36.0426 85.1662) (width 0.75) (layer "B.Cu") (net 6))
 (segment (start 7.8994 89.5604) (end 7.8994 83.6436) (width 0.75) (layer "F.Cu") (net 1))
 (segment (start 7.8994 83.6436) (end 7.8848 83.629) (width 0.75) (layer "F.Cu") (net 1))
 (via (at 7.8994 89.5604) (size 1.25) (drill 0.5) (layers "F.Cu" "B.Cu") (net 1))
 (segment (start 1.4986 39.4208) (end 1.4986 83.1596) (width 0.75) (layer "B.Cu") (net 1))
 (segment (start 1.4986 83.1596) (end 7.8994 89.5604) (width 0.75) (layer "B.Cu") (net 1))
 (segment (start 9.0972 36.322) (end 4.5974 36.322) (width 0.75) (layer "B.Cu") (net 1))
 (segment (start 4.5974 36.322) (end 1.4986 39.4208) (width 0.75) (layer "B.Cu") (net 1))
 (segment (start 9.8848 83.629) (end 9.8848 87.6512) (width 0.75) (layer "F.Cu") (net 2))
 (segment (start 9.8848 87.6512) (end 9.8298 87.7062) (width 0.75) (layer "F.Cu") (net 2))
 (via (at 9.8298 87.7062) (size 1.25) (drill 0.5) (layers "F.Cu" "B.Cu") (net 2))
 (segment (start 9.8298 87.7062) (end 8.0772 87.7062) (width 0.75) (layer "B.Cu") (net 2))
 (segment (start 2.667 82.296) (end 2.667 44.7294) (width 0.75) (layer "B.Cu") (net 2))
 (segment (start 2.667 44.7294) (end 7.7724 39.624) (width 0.75) (layer "B.Cu") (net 2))
 (segment (start 7.7724 39.624) (end 9.0972 39.624) (width 0.75) (layer "B.Cu") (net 2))
 (segment (start 8.0772 87.7062) (end 2.667 82.296) (width 0.75) (layer "B.Cu") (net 2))
 (segment (start 46.863 77.42892) (end 44.12952 77.42892) (width 0.75) (layer "F.Cu") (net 9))
 (segment (start 50.53628 81.1022) (end 46.863 77.42892) (width 0.75) (layer "F.Cu") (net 9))
 (segment (start 18.52036 73.02876) (end 5.18536 73.02876) (width 0.75) (layer "F.Cu") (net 9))
 (segment (start 5.18536 73.02876) (end 5.1562 72.9996) (width 0.75) (layer "F.Cu") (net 9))
 (segment (start 58.8602 82.6854) (end 57.277 81.1022) (width 0.75) (layer "F.Cu") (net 9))
 (segment (start 20.955 75.4634) (end 18.52036 73.02876) (width 0.75) (layer "F.Cu") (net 9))
 (segment (start 44.12952 77.42892) (end 42.164 75.4634) (width 0.75) (layer "F.Cu") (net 9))
 (segment (start 57.277 81.1022) (end 50.53628 81.1022) (width 0.75) (layer "F.Cu") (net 9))
 (segment (start 58.8602 85.05) (end 58.8602 82.6854) (width 0.75) (layer "F.Cu") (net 9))
 (segment (start 42.164 75.4634) (end 20.955 75.4634) (width 0.75) (layer "F.Cu") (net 9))
 (via (at 5.1562 72.9996) (size 1.25) (drill 0.5) (layers "F.Cu" "B.Cu") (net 9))
 (segment (start 5.1562 72.9996) (end 5.1562 46.867) (width 0.75) (layer "B.Cu") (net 9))
 (segment (start 5.1562 46.867) (end 9.0972 42.926) (width 0.75) (layer "B.Cu") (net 9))
 (segment (start 67.945 79.9592) (end 50.8254 79.9592) (width 0.75) (layer "F.Cu") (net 4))
 (segment (start 18.9738 72.07924) (end 14.25912 72.07924) (width 0.75) (layer "F.Cu") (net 4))
 (segment (start 68.8594 84.7742) (end 68.8594 80.8736) (width 0.75) (layer "F.Cu") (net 4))
 (segment (start 68.8602 85.05) (end 68.8602 84.775) (width 0.75) (layer "F.Cu") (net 4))
 (segment (start 47.3456 76.4794) (end 44.6786 76.4794) (width 0.75) (layer "F.Cu") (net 4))
 (segment (start 50.8254 79.9592) (end 47.3456 76.4794) (width 0.75) (layer "F.Cu") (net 4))
 (segment (start 68.8602 84.775) (end 68.8594 84.7742) (width 0.75) (layer "F.Cu") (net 4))
 (segment (start 68.8594 80.8736) (end 67.945 79.9592) (width 0.75) (layer "F.Cu") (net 4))
 (segment (start 21.39276 74.4982) (end 18.9738 72.07924) (width 0.75) (layer "F.Cu") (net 4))
 (segment (start 13.208 71.02812) (end 6.92448 71.02812) (width 0.75) (layer "F.Cu") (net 4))
 (segment (start 42.6974 74.4982) (end 21.39276 74.4982) (width 0.75) (layer "F.Cu") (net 4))
 (segment (start 14.25912 72.07924) (end 13.208 71.02812) (width 0.75) (layer "F.Cu") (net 4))
 (segment (start 44.6786 76.4794) (end 42.6974 74.4982) (width 0.75) (layer "F.Cu") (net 4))
 (segment (start 6.92448 71.02812) (end 6.9088 71.0438) (width 0.75) (layer "F.Cu") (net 4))
 (via (at 6.9088 71.0438) (size 1.25) (drill 0.5) (layers "F.Cu" "B.Cu") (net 4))
 (segment (start 6.9088 71.0438) (end 6.9088 48.4164) (width 0.75) (layer "B.Cu") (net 4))
 (segment (start 6.9088 48.4164) (end 9.0972 46.228) (width 0.75) (layer "B.Cu") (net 4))
 (segment (start 19.8882 88.0872) (end 19.8882 83.6324) (width 0.75) (layer "F.Cu") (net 10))
 (segment (start 19.8882 83.6324) (end 19.8848 83.629) (width 0.75) (layer "F.Cu") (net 10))
 (via (at 19.8882 88.0872) (size 1.25) (drill 0.5) (layers "F.Cu" "B.Cu") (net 10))
 (segment (start 18.0086 58.3906) (end 18.0086 86.995) (width 0.75) (layer "B.Cu") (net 10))
 (segment (start 19.1008 88.0872) (end 19.8882 88.0872) (width 0.75) (layer "B.Cu") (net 10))
 (segment (start 33.4732 42.926) (end 18.0086 58.3906) (width 0.75) (layer "B.Cu") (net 10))
 (segment (start 18.0086 86.995) (end 19.1008 88.0872) (width 0.75) (layer "B.Cu") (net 10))
 (segment (start 21.8694 83.6444) (end 21.8848 83.629) (width 0.75) (layer "F.Cu") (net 11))
 (segment (start 21.8694 88.138) (end 21.8694 83.6444) (width 0.75) (layer "F.Cu") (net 11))
 (via (at 21.8694 88.138) (size 1.25) (drill 0.5) (layers "F.Cu" "B.Cu") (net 11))
 (segment (start 23.5966 54.930803) (end 23.5966 87.5792) (width 0.75) (layer "B.Cu") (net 11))
 (segment (start 23.5966 87.5792) (end 23.0378 88.138) (width 0.75) (layer "B.Cu") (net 11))
 (segment (start 23.0378 88.138) (end 21.8694 88.138) (width 0.75) (layer "B.Cu") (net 11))
 (segment (start 32.299403 46.228) (end 23.5966 54.930803) (width 0.75) (layer "B.Cu") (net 11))
 (segment (start 33.4732 46.228) (end 32.299403 46.228) (width 0.75) (layer "B.Cu") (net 11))
 (segment (start 60.8602 85.05) (end 66.8602 85.05) (width 0.75) (layer "B.Cu") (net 3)))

